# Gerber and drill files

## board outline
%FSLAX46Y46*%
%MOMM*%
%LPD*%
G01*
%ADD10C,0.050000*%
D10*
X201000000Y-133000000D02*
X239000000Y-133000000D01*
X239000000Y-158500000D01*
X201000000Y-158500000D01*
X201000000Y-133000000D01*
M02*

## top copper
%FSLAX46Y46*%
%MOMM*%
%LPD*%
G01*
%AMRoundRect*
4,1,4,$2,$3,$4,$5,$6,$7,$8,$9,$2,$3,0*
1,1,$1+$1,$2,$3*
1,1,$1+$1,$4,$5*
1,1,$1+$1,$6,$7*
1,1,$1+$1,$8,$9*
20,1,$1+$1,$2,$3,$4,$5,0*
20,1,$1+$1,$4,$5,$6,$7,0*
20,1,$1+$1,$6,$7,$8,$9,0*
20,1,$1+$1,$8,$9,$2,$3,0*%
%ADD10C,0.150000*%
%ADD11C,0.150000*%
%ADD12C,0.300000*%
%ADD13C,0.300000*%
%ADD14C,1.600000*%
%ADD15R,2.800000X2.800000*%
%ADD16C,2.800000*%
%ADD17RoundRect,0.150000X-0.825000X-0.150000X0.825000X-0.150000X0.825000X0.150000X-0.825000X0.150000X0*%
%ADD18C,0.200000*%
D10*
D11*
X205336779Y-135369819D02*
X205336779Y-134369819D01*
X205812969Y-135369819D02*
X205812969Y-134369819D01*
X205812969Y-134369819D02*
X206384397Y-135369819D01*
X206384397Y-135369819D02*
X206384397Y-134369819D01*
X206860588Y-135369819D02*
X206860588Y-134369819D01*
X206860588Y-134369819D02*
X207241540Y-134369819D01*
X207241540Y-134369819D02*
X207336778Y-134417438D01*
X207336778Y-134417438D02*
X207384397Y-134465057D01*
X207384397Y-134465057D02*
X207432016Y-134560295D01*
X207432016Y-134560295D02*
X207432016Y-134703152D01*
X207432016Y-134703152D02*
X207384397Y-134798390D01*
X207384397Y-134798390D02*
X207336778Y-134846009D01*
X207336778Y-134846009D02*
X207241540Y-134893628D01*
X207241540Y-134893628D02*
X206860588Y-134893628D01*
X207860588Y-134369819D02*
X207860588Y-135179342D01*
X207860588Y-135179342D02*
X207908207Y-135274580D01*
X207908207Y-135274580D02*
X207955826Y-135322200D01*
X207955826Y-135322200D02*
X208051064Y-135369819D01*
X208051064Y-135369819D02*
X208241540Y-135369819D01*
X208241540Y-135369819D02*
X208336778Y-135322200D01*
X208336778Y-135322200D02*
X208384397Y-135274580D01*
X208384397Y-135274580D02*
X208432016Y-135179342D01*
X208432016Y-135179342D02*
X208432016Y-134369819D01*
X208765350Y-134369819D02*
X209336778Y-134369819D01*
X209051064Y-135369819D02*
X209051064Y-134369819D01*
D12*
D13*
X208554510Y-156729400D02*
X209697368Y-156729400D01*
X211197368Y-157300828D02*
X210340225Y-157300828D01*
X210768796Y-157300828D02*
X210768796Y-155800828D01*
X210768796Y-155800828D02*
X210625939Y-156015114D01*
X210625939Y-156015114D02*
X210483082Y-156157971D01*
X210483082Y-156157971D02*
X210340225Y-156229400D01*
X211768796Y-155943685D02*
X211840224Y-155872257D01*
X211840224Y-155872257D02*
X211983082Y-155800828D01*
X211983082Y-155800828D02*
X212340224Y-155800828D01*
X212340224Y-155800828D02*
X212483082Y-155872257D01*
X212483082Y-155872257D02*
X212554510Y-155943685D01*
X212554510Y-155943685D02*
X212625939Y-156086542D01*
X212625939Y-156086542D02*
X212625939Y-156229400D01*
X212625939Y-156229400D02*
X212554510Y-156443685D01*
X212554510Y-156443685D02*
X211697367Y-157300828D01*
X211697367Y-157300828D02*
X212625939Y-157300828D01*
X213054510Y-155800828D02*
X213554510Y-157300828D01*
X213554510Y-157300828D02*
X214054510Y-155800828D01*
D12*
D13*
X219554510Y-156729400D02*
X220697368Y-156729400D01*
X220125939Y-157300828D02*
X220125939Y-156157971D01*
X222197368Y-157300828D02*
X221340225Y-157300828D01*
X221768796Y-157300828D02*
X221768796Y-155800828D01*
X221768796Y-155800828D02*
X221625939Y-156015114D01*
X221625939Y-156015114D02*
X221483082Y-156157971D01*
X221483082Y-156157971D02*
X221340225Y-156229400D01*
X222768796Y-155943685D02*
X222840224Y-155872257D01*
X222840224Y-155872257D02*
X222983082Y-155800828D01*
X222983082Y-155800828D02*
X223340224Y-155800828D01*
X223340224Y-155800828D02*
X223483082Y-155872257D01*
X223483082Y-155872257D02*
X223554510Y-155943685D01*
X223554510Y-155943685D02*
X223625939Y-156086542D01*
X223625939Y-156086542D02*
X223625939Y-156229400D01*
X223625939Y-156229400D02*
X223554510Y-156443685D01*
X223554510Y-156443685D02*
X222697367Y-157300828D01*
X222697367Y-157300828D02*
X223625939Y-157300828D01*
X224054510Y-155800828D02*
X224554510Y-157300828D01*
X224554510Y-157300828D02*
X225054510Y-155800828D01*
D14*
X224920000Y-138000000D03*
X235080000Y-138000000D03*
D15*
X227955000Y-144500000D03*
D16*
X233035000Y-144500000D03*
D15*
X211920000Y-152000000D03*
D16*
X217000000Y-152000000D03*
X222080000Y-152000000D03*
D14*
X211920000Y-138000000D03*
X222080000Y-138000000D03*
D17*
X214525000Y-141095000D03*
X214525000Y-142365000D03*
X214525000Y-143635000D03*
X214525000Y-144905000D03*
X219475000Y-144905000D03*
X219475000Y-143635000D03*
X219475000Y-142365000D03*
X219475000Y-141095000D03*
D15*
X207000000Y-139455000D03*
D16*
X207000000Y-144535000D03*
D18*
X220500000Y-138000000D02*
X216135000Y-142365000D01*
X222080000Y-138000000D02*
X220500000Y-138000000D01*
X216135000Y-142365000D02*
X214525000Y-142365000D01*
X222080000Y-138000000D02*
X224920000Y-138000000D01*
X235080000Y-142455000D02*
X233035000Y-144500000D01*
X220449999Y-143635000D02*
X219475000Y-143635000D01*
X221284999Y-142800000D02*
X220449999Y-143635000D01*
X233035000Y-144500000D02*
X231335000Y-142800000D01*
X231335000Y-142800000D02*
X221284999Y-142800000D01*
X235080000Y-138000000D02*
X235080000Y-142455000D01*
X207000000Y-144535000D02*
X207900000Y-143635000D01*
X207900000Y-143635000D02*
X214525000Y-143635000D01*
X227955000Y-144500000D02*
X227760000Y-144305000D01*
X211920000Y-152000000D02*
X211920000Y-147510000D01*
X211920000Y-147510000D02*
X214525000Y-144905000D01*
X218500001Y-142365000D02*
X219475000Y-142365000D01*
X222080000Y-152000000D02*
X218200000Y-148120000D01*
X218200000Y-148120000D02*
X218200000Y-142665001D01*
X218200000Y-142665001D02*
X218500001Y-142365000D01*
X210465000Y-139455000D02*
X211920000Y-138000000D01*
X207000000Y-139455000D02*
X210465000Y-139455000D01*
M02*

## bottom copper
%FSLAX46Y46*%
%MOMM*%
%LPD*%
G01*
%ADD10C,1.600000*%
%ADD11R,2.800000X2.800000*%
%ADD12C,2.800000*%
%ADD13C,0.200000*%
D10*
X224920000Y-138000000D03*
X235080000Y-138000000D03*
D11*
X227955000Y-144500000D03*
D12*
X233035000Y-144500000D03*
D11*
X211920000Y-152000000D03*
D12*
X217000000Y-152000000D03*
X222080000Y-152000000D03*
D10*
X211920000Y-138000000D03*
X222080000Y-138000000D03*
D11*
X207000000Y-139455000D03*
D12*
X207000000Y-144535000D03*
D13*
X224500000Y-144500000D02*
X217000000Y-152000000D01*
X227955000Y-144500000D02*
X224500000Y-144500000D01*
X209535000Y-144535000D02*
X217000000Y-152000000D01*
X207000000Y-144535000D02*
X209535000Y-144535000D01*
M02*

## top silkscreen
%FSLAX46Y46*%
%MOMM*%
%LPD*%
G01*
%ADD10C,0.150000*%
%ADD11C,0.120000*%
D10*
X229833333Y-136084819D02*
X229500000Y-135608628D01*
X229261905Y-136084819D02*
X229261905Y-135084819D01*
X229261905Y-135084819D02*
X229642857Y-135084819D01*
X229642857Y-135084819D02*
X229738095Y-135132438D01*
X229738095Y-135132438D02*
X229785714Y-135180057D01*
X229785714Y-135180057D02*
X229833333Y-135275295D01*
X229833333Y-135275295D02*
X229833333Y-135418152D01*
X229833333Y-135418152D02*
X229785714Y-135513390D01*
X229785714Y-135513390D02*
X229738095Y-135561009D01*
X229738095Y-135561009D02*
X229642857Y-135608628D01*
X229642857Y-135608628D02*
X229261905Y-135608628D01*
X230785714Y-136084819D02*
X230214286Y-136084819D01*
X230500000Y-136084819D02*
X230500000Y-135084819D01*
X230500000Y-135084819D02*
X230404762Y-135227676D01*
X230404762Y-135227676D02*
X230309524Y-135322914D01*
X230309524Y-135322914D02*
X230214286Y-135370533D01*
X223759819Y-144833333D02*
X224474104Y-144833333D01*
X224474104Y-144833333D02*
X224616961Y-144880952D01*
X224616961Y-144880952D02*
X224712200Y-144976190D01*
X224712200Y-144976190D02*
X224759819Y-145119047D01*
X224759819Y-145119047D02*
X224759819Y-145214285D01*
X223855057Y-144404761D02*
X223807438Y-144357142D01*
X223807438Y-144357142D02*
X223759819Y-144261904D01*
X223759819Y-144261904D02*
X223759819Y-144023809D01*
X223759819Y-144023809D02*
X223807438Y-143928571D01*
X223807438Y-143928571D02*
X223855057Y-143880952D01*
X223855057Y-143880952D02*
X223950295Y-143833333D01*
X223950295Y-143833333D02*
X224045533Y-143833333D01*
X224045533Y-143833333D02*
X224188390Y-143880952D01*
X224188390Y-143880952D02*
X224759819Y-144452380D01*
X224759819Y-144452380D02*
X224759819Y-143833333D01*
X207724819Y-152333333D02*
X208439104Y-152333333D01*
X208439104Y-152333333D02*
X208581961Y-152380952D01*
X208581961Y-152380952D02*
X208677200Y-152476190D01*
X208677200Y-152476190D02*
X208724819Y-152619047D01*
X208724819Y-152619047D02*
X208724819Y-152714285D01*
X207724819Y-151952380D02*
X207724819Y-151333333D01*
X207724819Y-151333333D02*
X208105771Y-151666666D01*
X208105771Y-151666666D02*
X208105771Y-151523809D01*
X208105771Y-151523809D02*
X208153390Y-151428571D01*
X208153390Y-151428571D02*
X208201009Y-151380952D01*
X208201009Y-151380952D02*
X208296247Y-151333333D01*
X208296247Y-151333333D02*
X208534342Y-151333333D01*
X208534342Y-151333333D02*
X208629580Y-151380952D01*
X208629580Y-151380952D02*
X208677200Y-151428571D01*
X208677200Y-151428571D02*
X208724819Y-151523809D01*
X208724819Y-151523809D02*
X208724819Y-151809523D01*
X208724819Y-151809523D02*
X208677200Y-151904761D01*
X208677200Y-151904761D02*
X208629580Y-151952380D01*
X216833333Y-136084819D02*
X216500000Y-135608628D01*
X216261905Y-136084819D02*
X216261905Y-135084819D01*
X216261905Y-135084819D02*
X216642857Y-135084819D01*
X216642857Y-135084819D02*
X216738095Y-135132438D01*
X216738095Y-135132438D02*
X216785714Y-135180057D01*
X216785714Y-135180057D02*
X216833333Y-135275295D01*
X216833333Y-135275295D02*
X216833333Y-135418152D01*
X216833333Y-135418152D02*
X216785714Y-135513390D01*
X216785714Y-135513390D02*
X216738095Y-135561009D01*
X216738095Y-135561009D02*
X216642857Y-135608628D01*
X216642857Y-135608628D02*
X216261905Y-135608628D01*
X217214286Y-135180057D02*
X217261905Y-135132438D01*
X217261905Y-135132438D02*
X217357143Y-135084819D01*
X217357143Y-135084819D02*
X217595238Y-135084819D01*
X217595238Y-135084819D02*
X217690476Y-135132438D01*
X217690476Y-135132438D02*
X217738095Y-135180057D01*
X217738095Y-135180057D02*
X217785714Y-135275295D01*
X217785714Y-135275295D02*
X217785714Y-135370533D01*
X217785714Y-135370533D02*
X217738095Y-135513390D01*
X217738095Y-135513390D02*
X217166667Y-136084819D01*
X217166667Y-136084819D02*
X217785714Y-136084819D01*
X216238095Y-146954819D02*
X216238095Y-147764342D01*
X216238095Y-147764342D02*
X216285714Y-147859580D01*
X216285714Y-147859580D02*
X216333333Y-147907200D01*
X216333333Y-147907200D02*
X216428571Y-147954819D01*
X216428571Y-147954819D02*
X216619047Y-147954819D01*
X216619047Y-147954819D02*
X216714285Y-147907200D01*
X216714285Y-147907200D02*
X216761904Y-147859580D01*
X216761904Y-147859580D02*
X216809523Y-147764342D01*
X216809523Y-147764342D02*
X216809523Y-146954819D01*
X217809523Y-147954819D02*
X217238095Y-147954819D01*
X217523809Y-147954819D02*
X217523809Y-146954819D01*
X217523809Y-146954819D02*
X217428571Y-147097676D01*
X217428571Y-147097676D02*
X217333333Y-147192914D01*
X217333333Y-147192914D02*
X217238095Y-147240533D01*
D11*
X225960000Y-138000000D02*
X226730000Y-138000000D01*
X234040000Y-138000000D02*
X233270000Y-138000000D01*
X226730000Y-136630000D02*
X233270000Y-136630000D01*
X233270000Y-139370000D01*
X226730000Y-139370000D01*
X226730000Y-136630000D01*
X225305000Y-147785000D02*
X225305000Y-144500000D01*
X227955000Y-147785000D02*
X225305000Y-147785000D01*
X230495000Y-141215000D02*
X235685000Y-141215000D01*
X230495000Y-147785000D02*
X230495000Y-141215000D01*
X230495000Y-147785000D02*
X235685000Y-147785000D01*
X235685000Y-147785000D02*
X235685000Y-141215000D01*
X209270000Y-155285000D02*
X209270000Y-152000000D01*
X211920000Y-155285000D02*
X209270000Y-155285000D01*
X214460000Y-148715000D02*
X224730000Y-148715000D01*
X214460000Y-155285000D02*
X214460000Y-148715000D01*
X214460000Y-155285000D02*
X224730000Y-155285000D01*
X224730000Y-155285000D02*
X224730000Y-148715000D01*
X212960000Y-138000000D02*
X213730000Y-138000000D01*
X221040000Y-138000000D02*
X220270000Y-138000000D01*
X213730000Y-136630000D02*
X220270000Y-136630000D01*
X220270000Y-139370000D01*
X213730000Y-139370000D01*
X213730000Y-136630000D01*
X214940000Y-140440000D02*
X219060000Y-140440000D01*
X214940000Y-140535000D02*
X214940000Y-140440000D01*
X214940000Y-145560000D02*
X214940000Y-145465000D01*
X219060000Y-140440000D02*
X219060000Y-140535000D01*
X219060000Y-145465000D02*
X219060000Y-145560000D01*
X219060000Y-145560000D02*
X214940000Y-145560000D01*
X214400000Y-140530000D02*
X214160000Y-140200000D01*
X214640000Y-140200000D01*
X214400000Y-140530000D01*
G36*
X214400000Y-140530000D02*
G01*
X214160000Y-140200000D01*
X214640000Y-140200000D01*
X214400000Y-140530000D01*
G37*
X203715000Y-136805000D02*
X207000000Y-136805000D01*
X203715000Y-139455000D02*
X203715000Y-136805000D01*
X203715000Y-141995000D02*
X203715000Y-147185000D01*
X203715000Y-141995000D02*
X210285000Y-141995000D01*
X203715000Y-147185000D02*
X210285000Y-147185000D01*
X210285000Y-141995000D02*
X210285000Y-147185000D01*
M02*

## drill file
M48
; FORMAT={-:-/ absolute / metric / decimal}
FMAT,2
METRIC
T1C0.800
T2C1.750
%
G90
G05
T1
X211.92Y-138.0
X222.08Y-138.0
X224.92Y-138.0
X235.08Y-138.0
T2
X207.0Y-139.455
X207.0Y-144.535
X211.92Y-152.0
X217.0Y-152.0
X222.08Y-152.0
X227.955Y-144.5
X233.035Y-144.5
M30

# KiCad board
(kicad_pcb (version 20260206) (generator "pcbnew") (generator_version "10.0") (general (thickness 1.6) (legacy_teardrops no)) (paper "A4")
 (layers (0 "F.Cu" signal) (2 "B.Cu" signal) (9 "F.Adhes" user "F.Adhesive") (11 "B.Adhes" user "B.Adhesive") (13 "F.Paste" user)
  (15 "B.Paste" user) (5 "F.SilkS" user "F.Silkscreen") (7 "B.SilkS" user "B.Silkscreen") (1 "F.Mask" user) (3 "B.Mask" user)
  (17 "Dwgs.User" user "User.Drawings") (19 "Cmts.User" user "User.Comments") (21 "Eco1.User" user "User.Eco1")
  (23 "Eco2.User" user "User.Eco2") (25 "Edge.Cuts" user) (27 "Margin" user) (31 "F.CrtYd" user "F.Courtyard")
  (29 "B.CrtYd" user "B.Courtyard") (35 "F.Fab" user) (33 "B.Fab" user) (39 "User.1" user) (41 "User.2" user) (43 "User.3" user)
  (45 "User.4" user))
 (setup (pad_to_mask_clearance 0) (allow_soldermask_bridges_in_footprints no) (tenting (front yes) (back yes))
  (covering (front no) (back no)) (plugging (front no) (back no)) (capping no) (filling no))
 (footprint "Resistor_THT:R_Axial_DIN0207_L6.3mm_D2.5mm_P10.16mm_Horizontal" (layer "F.Cu") (at 224.92 138)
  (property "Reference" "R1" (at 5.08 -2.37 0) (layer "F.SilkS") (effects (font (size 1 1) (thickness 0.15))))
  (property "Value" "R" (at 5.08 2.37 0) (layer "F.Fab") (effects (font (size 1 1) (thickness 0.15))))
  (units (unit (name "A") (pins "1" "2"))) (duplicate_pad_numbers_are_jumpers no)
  (fp_line (start 1.04 0) (end 1.81 0) (stroke (width 0.12) (type solid)) (layer "F.SilkS"))
  (fp_line (start 9.12 0) (end 8.35 0) (stroke (width 0.12) (type solid)) (layer "F.SilkS"))
  (fp_rect (start 1.81 -1.37) (end 8.35 1.37) (stroke (width 0.12) (type solid)) (fill no) (layer "F.SilkS"))
  (pad "1" thru_hole circle (at 0 0) (size 1.6 1.6) (drill 0.8) (layers "*.Cu" "*.Mask") (remove_unused_layers no) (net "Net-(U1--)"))
  (pad "2" thru_hole circle (at 10.16 0) (size 1.6 1.6) (drill 0.8) (layers "*.Cu" "*.Mask") (remove_unused_layers no)
   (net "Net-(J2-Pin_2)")))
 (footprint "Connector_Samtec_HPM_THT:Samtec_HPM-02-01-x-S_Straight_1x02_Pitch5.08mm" (layer "F.Cu") (at 227.955 144.5 90)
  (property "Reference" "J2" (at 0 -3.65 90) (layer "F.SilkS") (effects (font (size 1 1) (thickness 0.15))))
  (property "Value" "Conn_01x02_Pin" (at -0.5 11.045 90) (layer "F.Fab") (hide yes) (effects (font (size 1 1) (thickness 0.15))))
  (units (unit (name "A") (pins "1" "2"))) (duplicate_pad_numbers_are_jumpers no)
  (fp_line (start -3.285 -2.65) (end 0 -2.65) (stroke (width 0.12) (type solid)) (layer "F.SilkS"))
  (fp_line (start -3.285 0) (end -3.285 -2.65) (stroke (width 0.12) (type solid)) (layer "F.SilkS"))
  (fp_line (start 3.285 2.54) (end 3.285 7.73) (stroke (width 0.12) (type solid)) (layer "F.SilkS"))
  (fp_line (start -3.285 2.54) (end 3.285 2.54) (stroke (width 0.12) (type solid)) (layer "F.SilkS"))
  (fp_line (start -3.285 2.54) (end -3.285 7.73) (stroke (width 0.12) (type solid)) (layer "F.SilkS"))
  (fp_line (start -3.285 7.73) (end 3.285 7.73) (stroke (width 0.12) (type solid)) (layer "F.SilkS"))
  (pad "1" thru_hole rect (at 0 0 90) (size 2.8 2.8) (drill 1.75) (layers "*.Cu" "*.Mask") (remove_unused_layers no) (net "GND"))
  (pad "2" thru_hole circle (at 0 5.08 90) (size 2.8 2.8) (drill 1.75) (layers "*.Cu" "*.Mask") (remove_unused_layers no)
   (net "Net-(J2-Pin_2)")))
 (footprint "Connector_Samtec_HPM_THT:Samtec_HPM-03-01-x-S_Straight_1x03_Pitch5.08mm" (layer "F.Cu") (at 211.92 152 90)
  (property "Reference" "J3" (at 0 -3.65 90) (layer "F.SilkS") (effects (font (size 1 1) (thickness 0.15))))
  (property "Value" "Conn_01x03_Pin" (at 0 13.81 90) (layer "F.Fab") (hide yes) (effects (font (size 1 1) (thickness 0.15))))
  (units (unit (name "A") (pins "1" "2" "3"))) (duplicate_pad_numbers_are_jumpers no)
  (fp_line (start -3.285 -2.65) (end 0 -2.65) (stroke (width 0.12) (type solid)) (layer "F.SilkS"))
  (fp_line (start -3.285 0) (end -3.285 -2.65) (stroke (width 0.12) (type solid)) (layer "F.SilkS"))
  (fp_line (start 3.285 2.54) (end 3.285 12.81) (stroke (width 0.12) (type solid)) (layer "F.SilkS"))
  (fp_line (start -3.285 2.54) (end 3.285 2.54) (stroke (width 0.12) (type solid)) (layer "F.SilkS"))
  (fp_line (start -3.285 2.54) (end -3.285 12.81) (stroke (width 0.12) (type solid)) (layer "F.SilkS"))
  (fp_line (start -3.285 12.81) (end 3.285 12.81) (stroke (width 0.12) (type solid)) (layer "F.SilkS"))
  (pad "1" thru_hole rect (at 0 0 90) (size 2.8 2.8) (drill 1.75) (layers "*.Cu" "*.Mask") (remove_unused_layers no) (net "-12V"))
  (pad "2" thru_hole circle (at 0 5.08 90) (size 2.8 2.8) (drill 1.75) (layers "*.Cu" "*.Mask") (remove_unused_layers no) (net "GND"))
  (pad "3" thru_hole circle (at 0 10.16 90) (size 2.8 2.8) (drill 1.75) (layers "*.Cu" "*.Mask") (remove_unused_layers no) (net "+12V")))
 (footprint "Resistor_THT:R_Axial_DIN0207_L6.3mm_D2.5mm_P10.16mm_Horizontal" (layer "F.Cu") (at 211.92 138)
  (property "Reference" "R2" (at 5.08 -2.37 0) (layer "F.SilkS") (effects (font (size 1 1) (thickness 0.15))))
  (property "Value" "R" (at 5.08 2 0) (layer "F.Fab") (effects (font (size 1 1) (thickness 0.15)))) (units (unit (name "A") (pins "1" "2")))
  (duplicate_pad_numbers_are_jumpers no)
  (fp_line (start 1.04 0) (end 1.81 0) (stroke (width 0.12) (type solid)) (layer "F.SilkS"))
  (fp_line (start 9.12 0) (end 8.35 0) (stroke (width 0.12) (type solid)) (layer "F.SilkS"))
  (fp_rect (start 1.81 -1.37) (end 8.35 1.37) (stroke (width 0.12) (type solid)) (fill no) (layer "F.SilkS"))
  (pad "1" thru_hole circle (at 0 0) (size 1.6 1.6) (drill 0.8) (layers "*.Cu" "*.Mask") (remove_unused_layers no) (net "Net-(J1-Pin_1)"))
  (pad "2" thru_hole circle (at 10.16 0) (size 1.6 1.6) (drill 0.8) (layers "*.Cu" "*.Mask") (remove_unused_layers no) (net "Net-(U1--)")))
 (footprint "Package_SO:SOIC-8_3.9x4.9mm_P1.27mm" (layer "F.Cu") (at 217 143)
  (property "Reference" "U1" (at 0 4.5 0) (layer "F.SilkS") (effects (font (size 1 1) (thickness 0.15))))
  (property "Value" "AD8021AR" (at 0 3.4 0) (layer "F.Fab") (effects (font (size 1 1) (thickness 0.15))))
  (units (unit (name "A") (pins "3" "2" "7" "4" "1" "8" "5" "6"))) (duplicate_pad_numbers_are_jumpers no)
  (fp_line (start -2.06 -2.56) (end 2.06 -2.56) (stroke (width 0.12) (type solid)) (layer "F.SilkS"))
  (fp_line (start -2.06 -2.465) (end -2.06 -2.56) (stroke (width 0.12) (type solid)) (layer "F.SilkS"))
  (fp_line (start -2.06 2.56) (end -2.06 2.465) (stroke (width 0.12) (type solid)) (layer "F.SilkS"))
  (fp_line (start 2.06 -2.56) (end 2.06 -2.465) (stroke (width 0.12) (type solid)) (layer "F.SilkS"))
  (fp_line (start 2.06 2.465) (end 2.06 2.56) (stroke (width 0.12) (type solid)) (layer "F.SilkS"))
  (fp_line (start 2.06 2.56) (end -2.06 2.56) (stroke (width 0.12) (type solid)) (layer "F.SilkS"))
  (fp_poly (pts (xy -2.6 -2.47) (xy -2.84 -2.8) (xy -2.36 -2.8)) (stroke (width 0.12) (type solid)) (fill yes) (layer "F.SilkS"))
  (pad "1" smd roundrect (at -2.475 -1.905) (size 1.95 0.6) (layers "F.Cu" "F.Mask" "F.Paste") (roundrect_rratio 0.25)
   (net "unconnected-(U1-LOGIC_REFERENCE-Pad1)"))
  (pad "2" smd roundrect (at -2.475 -0.635) (size 1.95 0.6) (layers "F.Cu" "F.Mask" "F.Paste") (roundrect_rratio 0.25) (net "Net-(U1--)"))
  (pad "3" smd roundrect (at -2.475 0.635) (size 1.95 0.6) (layers "F.Cu" "F.Mask" "F.Paste") (roundrect_rratio 0.25) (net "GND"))
  (pad "4" smd roundrect (at -2.475 1.905) (size 1.95 0.6) (layers "F.Cu" "F.Mask" "F.Paste") (roundrect_rratio 0.25) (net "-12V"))
  (pad "5" smd roundrect (at 2.475 1.905) (size 1.95 0.6) (layers "F.Cu" "F.Mask" "F.Paste") (roundrect_rratio 0.25)
   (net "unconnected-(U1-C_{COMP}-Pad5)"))
  (pad "6" smd roundrect (at 2.475 0.635) (size 1.95 0.6) (layers "F.Cu" "F.Mask" "F.Paste") (roundrect_rratio 0.25) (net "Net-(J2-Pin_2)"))
  (pad "7" smd roundrect (at 2.475 -0.635) (size 1.95 0.6) (layers "F.Cu" "F.Mask" "F.Paste") (roundrect_rratio 0.25) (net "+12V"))
  (pad "8" smd roundrect (at 2.475 -1.905) (size 1.95 0.6) (layers "F.Cu" "F.Mask" "F.Paste") (roundrect_rratio 0.25)
   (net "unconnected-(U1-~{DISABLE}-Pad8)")))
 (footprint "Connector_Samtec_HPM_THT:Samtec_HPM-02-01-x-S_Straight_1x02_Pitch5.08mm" (layer "F.Cu") (at 207 139.455)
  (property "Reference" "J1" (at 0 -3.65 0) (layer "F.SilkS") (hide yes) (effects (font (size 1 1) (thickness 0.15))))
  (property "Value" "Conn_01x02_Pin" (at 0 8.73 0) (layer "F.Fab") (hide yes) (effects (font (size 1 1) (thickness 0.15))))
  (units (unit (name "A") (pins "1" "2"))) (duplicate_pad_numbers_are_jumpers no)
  (fp_line (start -3.285 -2.65) (end 0 -2.65) (stroke (width 0.12) (type solid)) (layer "F.SilkS"))
  (fp_line (start -3.285 0) (end -3.285 -2.65) (stroke (width 0.12) (type solid)) (layer "F.SilkS"))
  (fp_line (start -3.285 2.54) (end -3.285 7.73) (stroke (width 0.12) (type solid)) (layer "F.SilkS"))
  (fp_line (start -3.285 2.54) (end 3.285 2.54) (stroke (width 0.12) (type solid)) (layer "F.SilkS"))
  (fp_line (start -3.285 7.73) (end 3.285 7.73) (stroke (width 0.12) (type solid)) (layer "F.SilkS"))
  (fp_line (start 3.285 2.54) (end 3.285 7.73) (stroke (width 0.12) (type solid)) (layer "F.SilkS"))
  (pad "1" thru_hole rect (at 0 0) (size 2.8 2.8) (drill 1.75) (layers "*.Cu" "*.Mask") (remove_unused_layers no) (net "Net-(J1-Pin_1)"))
  (pad "2" thru_hole circle (at 0 5.08) (size 2.8 2.8) (drill 1.75) (layers "*.Cu" "*.Mask") (remove_unused_layers no) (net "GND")))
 (gr_rect (start 201 133) (end 239 158.5) (stroke (width 0.05) (type default)) (fill no) (layer "Edge.Cuts"))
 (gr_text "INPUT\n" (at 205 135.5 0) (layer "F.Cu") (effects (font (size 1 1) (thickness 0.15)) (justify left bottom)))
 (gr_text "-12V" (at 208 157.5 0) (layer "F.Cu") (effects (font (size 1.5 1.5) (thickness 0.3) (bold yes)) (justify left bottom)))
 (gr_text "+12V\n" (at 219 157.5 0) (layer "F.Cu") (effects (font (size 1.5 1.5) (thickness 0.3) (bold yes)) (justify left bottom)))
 (segment (start 220.5 138) (end 216.135 142.365) (width 0.2) (layer "F.Cu") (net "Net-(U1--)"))
 (segment (start 222.08 138) (end 220.5 138) (width 0.2) (layer "F.Cu") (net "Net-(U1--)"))
 (segment (start 216.135 142.365) (end 214.525 142.365) (width 0.2) (layer "F.Cu") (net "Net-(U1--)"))
 (segment (start 222.08 138) (end 224.92 138) (width 0.2) (layer "F.Cu") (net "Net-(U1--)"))
 (segment (start 235.08 142.455) (end 233.035 144.5) (width 0.2) (layer "F.Cu") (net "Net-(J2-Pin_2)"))
 (segment (start 220.449999 143.635) (end 219.475 143.635) (width 0.2) (layer "F.Cu") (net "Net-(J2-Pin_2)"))
 (segment (start 221.284999 142.8) (end 220.449999 143.635) (width 0.2) (layer "F.Cu") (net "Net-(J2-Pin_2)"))
 (segment (start 233.035 144.5) (end 231.335 142.8) (width 0.2) (layer "F.Cu") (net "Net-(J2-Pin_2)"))
 (segment (start 231.335 142.8) (end 221.284999 142.8) (width 0.2) (layer "F.Cu") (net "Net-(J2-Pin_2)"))
 (segment (start 235.08 138) (end 235.08 142.455) (width 0.2) (layer "F.Cu") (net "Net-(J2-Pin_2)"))
 (segment (start 207 144.535) (end 207.9 143.635) (width 0.2) (layer "F.Cu") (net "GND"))
 (segment (start 207.9 143.635) (end 214.525 143.635) (width 0.2) (layer "F.Cu") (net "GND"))
 (segment (start 227.955 144.5) (end 227.76 144.305) (width 0.2) (layer "F.Cu") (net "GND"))
 (segment (start 224.5 144.5) (end 217 152) (width 0.2) (layer "B.Cu") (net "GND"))
 (segment (start 227.955 144.5) (end 224.5 144.5) (width 0.2) (layer "B.Cu") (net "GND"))
 (segment (start 209.535 144.535) (end 217 152) (width 0.2) (layer "B.Cu") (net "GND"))
 (segment (start 207 144.535) (end 209.535 144.535) (width 0.2) (layer "B.Cu") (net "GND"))
 (segment (start 211.92 152) (end 211.92 147.51) (width 0.2) (layer "F.Cu") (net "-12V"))
 (segment (start 211.92 147.51) (end 214.525 144.905) (width 0.2) (layer "F.Cu") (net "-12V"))
 (segment (start 218.500001 142.365) (end 219.475 142.365) (width 0.2) (layer "F.Cu") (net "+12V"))
 (segment (start 222.08 152) (end 218.2 148.12) (width 0.2) (layer "F.Cu") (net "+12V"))
 (segment (start 218.2 148.12) (end 218.2 142.665001) (width 0.2) (layer "F.Cu") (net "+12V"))
 (segment (start 218.2 142.665001) (end 218.500001 142.365) (width 0.2) (layer "F.Cu") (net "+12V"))
 (segment (start 210.465 139.455) (end 211.92 138) (width 0.2) (layer "F.Cu") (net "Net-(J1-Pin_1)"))
 (segment (start 207 139.455) (end 210.465 139.455) (width 0.2) (layer "F.Cu") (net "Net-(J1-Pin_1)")))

